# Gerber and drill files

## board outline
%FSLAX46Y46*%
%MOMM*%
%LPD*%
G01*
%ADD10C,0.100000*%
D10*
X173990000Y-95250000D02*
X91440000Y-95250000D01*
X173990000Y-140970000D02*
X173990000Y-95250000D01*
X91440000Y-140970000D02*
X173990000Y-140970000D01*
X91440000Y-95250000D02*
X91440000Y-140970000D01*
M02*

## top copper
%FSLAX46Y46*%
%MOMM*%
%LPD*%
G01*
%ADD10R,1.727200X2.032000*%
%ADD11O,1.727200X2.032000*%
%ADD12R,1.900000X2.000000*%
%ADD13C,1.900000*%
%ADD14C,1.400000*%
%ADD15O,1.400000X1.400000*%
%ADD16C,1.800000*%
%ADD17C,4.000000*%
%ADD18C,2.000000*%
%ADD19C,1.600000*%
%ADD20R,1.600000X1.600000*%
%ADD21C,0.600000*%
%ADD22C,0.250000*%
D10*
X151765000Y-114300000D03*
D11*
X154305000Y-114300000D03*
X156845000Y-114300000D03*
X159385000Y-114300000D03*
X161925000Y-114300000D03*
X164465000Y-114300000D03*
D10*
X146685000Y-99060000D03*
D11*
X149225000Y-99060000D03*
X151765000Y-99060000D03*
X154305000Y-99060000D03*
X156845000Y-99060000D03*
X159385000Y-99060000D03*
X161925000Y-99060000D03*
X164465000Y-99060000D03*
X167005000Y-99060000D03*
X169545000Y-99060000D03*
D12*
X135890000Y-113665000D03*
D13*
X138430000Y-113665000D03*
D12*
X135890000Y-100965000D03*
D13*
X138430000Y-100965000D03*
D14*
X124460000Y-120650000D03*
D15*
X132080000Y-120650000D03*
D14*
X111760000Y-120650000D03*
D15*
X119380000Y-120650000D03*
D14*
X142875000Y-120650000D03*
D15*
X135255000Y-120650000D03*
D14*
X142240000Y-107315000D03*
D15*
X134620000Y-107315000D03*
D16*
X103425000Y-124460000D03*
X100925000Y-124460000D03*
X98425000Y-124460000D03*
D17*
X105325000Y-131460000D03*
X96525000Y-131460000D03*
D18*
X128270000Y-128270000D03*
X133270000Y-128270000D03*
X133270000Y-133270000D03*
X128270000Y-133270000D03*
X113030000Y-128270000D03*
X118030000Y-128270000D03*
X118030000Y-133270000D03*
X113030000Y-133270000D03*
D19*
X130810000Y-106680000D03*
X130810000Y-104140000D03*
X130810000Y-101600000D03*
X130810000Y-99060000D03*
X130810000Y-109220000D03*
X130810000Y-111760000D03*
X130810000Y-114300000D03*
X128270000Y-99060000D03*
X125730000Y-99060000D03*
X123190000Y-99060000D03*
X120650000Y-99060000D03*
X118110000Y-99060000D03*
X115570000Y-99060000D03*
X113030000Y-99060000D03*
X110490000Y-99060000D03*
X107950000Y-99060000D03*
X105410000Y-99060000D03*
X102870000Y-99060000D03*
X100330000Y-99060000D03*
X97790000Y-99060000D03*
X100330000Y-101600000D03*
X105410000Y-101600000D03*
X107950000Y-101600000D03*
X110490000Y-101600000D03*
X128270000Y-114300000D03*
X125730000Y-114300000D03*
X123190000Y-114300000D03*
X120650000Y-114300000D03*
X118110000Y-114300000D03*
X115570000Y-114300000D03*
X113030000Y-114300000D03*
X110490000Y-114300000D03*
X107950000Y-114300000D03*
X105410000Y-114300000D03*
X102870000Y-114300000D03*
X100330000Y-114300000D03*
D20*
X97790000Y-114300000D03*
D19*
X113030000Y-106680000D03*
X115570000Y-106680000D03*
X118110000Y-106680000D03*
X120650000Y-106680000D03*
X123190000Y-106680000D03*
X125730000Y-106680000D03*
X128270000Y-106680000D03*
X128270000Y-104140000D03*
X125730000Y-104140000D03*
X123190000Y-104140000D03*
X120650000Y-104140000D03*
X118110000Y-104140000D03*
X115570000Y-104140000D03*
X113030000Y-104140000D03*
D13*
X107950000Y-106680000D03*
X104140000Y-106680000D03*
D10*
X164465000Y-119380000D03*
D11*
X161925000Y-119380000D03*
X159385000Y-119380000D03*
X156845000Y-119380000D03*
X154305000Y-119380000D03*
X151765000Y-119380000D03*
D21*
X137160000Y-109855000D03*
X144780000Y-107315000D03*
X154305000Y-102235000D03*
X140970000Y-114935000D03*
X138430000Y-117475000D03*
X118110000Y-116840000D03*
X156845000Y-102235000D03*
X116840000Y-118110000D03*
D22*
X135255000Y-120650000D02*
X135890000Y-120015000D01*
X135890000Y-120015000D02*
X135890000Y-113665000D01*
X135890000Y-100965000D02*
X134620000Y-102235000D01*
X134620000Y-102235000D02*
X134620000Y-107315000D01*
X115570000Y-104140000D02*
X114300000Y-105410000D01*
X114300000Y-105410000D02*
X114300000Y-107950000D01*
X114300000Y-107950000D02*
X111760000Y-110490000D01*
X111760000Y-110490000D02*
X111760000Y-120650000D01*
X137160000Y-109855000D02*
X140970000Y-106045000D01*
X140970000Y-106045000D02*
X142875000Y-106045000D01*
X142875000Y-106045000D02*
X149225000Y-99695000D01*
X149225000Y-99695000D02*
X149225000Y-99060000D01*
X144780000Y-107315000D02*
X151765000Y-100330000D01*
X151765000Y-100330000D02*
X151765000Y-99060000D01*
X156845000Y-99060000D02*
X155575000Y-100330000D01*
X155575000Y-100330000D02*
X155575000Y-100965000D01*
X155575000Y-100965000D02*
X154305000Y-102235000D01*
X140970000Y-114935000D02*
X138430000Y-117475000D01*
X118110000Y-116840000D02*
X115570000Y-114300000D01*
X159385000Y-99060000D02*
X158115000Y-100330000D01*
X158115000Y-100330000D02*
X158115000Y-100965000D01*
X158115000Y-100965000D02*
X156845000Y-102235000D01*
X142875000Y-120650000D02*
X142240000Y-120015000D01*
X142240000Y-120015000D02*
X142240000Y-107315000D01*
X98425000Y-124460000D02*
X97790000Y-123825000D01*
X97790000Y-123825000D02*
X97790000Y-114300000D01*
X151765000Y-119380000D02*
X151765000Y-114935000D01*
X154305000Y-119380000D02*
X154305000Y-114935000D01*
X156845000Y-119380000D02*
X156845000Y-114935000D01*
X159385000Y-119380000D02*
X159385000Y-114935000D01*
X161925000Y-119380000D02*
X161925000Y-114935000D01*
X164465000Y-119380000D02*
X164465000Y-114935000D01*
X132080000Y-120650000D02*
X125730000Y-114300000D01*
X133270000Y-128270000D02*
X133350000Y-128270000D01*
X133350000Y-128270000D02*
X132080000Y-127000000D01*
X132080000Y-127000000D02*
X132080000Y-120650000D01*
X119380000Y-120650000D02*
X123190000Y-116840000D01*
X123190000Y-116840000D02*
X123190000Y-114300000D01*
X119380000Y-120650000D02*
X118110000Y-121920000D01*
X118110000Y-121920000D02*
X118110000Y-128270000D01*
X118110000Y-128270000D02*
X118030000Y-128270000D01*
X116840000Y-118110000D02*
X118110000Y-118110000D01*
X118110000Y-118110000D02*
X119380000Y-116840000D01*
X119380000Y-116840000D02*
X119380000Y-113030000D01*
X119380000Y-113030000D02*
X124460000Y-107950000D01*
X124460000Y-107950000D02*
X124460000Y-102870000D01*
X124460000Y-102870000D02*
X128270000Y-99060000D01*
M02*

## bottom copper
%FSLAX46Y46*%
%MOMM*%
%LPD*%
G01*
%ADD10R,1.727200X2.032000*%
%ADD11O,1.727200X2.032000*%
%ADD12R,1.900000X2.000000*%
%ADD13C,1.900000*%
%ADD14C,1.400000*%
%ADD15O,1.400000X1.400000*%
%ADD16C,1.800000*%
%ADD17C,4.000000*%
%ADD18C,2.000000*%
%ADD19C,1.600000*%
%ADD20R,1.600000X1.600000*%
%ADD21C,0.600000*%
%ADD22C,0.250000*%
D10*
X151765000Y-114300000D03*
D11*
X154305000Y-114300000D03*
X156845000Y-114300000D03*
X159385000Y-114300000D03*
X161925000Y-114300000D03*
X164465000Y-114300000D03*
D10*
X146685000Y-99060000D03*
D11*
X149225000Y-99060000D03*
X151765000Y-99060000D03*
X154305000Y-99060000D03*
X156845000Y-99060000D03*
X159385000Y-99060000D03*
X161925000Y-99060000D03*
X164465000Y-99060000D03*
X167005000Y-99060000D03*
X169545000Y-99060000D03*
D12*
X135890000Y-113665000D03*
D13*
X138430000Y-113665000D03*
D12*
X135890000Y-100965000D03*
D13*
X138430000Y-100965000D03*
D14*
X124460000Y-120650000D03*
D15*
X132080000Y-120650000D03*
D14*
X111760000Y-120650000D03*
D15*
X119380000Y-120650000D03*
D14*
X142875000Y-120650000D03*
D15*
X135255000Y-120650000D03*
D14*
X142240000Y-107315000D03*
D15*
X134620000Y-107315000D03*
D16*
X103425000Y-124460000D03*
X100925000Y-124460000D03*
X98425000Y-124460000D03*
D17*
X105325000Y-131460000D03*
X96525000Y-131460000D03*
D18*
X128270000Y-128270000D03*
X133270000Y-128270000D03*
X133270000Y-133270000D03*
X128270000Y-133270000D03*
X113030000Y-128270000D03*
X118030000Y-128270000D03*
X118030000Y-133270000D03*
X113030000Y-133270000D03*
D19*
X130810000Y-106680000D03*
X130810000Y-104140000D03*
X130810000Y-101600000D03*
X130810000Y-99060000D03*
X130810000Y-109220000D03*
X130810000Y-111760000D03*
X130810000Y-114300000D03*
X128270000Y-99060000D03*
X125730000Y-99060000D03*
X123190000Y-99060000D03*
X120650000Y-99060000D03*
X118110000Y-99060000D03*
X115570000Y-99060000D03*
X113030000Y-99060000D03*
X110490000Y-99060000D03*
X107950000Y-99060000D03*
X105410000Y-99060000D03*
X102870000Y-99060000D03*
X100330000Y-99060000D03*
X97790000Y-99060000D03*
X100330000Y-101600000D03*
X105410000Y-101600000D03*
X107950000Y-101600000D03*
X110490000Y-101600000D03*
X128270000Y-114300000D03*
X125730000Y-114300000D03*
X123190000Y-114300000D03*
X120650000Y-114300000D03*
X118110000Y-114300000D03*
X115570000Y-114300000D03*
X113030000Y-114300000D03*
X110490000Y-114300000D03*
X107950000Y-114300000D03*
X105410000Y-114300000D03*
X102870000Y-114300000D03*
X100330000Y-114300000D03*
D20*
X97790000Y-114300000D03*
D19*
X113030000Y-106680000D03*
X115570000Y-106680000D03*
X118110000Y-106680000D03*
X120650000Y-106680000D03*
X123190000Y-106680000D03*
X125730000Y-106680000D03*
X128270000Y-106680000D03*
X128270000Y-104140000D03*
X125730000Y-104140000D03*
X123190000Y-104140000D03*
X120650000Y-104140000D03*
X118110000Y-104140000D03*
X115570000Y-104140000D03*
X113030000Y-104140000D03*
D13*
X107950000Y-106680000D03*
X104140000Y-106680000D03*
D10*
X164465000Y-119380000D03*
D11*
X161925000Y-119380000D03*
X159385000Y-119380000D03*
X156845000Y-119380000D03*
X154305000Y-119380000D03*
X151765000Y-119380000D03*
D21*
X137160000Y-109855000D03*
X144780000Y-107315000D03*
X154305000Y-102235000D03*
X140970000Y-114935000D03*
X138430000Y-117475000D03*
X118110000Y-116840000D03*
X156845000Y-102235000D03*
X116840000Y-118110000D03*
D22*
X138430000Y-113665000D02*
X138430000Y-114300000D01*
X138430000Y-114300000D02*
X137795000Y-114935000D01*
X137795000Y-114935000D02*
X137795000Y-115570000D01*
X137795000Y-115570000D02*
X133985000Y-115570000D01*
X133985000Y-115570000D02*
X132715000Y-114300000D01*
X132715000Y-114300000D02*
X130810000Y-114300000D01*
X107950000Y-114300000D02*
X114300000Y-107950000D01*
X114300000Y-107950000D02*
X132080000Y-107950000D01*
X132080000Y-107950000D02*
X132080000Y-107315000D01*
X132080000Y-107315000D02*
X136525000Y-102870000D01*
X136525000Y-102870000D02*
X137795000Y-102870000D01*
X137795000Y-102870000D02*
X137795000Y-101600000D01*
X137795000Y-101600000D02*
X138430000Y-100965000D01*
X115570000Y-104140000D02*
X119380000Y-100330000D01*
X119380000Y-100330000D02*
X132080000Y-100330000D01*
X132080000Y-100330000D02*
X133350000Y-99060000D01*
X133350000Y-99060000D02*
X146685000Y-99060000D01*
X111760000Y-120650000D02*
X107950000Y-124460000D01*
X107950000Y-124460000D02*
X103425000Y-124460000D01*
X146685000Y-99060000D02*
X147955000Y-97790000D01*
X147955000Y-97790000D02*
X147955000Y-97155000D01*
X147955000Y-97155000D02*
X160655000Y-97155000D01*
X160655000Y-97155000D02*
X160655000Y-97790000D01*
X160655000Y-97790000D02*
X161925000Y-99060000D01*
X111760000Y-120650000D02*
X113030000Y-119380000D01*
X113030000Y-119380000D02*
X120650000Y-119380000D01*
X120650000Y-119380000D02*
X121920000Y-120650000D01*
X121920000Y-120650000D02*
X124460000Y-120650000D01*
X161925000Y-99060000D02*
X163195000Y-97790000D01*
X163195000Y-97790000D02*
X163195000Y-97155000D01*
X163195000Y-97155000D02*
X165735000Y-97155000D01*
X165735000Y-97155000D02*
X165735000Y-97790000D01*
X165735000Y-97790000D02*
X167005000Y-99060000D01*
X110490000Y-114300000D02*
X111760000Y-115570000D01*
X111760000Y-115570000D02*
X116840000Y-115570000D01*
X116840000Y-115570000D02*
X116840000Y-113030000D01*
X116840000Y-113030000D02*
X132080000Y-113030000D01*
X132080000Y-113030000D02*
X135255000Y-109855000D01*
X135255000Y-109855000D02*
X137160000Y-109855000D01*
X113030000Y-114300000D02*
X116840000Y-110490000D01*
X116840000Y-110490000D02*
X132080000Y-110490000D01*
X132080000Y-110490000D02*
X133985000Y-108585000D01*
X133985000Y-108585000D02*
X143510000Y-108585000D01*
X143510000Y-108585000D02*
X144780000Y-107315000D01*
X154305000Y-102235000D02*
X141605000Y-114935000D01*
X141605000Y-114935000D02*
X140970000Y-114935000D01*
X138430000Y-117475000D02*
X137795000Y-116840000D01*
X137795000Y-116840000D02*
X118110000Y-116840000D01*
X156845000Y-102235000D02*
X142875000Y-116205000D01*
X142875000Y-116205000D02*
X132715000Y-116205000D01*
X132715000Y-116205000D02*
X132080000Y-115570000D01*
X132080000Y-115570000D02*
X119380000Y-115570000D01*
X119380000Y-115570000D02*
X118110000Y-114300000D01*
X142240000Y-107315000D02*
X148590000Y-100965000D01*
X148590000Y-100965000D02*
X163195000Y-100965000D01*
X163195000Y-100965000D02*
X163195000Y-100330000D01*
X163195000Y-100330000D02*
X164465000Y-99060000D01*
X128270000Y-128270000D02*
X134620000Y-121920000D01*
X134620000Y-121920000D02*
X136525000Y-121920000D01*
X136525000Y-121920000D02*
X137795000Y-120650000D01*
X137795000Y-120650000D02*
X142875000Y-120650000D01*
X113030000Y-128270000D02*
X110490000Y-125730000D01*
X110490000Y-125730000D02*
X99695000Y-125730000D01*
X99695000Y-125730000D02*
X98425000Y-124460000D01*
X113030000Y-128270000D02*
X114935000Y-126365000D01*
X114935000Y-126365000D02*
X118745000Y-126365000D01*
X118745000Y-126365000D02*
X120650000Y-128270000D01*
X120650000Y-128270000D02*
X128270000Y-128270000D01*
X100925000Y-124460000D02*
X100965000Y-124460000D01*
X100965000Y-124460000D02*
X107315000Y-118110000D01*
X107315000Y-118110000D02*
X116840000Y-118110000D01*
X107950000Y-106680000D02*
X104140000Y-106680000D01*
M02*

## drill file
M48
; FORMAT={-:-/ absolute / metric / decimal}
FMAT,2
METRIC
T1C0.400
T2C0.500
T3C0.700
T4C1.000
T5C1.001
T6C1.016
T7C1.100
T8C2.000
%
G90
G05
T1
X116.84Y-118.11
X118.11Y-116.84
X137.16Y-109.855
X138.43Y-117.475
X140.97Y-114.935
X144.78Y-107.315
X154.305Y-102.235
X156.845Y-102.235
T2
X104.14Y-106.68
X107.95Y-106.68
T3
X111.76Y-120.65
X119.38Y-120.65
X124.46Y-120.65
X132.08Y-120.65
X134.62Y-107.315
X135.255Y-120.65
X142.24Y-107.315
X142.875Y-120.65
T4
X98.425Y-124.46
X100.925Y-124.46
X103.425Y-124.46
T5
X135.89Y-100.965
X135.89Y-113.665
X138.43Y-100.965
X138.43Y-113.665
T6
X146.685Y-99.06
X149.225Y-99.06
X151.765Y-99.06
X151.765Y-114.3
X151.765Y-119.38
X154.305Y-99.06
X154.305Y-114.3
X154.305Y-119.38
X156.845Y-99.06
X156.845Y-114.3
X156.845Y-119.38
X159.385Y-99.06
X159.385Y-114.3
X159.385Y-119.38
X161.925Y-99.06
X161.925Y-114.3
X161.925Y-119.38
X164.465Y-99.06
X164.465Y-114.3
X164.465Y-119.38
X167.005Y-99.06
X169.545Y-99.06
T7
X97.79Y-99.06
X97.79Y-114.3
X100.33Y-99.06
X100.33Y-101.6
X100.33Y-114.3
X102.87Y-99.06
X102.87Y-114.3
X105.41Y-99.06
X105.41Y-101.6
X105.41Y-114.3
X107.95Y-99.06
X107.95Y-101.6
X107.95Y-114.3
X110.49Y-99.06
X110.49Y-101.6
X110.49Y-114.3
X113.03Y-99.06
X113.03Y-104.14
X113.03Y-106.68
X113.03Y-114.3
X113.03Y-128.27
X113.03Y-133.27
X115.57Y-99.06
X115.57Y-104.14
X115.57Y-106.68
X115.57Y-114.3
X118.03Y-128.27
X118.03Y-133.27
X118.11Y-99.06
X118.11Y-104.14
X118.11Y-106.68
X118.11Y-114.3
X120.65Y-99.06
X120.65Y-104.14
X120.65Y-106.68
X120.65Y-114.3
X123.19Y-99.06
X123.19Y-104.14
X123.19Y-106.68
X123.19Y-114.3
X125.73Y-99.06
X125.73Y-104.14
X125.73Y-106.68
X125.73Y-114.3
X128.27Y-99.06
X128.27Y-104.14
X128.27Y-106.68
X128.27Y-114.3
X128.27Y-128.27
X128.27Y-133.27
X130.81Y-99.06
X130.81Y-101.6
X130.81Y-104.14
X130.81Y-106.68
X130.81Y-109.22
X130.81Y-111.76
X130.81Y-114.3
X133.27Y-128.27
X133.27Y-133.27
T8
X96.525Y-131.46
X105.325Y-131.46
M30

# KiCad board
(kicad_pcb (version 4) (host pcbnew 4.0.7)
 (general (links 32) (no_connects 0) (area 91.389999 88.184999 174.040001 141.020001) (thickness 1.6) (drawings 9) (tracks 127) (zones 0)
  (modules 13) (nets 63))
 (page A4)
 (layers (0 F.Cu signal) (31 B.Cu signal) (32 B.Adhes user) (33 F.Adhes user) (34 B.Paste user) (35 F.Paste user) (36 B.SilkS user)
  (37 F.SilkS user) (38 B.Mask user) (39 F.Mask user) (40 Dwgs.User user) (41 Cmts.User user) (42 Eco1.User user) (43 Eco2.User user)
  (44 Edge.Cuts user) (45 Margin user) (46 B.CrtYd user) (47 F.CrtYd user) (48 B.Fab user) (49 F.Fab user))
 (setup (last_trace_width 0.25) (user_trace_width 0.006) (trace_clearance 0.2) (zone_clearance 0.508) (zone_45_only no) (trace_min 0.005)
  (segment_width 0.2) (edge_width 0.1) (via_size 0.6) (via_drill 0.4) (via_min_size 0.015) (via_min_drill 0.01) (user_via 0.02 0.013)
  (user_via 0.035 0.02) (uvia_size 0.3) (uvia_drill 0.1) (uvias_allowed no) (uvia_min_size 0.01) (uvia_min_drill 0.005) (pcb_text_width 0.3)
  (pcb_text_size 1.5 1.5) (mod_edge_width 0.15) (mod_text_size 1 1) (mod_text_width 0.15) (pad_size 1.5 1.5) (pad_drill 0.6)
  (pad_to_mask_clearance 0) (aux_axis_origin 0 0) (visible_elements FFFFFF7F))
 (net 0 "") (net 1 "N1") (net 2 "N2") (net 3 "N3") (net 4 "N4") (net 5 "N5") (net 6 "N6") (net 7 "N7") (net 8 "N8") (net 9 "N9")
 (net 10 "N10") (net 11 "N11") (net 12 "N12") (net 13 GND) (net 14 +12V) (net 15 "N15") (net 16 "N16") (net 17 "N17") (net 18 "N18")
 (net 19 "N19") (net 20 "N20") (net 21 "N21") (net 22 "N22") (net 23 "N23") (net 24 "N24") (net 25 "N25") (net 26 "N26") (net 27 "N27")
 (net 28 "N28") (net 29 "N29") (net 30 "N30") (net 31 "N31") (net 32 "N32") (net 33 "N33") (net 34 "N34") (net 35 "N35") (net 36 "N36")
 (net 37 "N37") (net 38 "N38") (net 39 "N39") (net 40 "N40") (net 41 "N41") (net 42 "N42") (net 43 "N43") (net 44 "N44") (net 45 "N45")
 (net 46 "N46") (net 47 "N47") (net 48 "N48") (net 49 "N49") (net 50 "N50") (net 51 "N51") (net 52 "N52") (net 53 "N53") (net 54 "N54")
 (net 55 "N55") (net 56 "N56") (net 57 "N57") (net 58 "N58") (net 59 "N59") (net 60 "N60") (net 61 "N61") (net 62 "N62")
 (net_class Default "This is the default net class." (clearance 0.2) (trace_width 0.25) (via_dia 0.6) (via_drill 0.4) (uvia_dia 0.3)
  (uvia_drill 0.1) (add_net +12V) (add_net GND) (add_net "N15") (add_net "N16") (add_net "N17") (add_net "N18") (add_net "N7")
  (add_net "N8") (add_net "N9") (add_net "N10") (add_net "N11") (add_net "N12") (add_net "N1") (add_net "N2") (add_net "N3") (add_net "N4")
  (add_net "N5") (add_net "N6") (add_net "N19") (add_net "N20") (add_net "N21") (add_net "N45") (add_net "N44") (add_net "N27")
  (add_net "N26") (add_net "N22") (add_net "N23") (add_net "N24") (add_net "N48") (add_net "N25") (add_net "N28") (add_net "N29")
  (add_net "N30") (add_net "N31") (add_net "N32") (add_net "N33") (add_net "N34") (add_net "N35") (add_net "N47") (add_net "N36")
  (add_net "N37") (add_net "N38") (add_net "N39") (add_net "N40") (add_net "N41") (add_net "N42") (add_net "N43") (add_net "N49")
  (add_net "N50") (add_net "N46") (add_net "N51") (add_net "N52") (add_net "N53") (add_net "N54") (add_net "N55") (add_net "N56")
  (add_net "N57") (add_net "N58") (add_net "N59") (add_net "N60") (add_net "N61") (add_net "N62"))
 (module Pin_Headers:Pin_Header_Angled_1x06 (layer F.Cu) (at 151.765 114.3 90)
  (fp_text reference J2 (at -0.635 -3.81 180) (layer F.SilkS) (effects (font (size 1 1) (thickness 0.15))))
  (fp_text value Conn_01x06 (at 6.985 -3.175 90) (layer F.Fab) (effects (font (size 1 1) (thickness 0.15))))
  (pad 1 thru_hole rect (at 0 0 90) (size 2.032 1.7272) (drill 1.016) (layers *.Cu *.Mask) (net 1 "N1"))
  (pad 2 thru_hole oval (at 0 2.54 90) (size 2.032 1.7272) (drill 1.016) (layers *.Cu *.Mask) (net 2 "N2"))
  (pad 3 thru_hole oval (at 0 5.08 90) (size 2.032 1.7272) (drill 1.016) (layers *.Cu *.Mask) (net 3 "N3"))
  (pad 4 thru_hole oval (at 0 7.62 90) (size 2.032 1.7272) (drill 1.016) (layers *.Cu *.Mask) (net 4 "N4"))
  (pad 5 thru_hole oval (at 0 10.16 90) (size 2.032 1.7272) (drill 1.016) (layers *.Cu *.Mask) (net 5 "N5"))
  (pad 6 thru_hole oval (at 0 12.7 90) (size 2.032 1.7272) (drill 1.016) (layers *.Cu *.Mask) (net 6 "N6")))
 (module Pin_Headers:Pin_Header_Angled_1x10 (layer F.Cu) (at 146.685 99.06 90)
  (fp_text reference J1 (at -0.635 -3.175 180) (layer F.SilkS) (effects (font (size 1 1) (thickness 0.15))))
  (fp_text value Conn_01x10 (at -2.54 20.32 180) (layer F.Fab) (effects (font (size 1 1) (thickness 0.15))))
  (pad 1 thru_hole rect (at 0 0 90) (size 2.032 1.7272) (drill 1.016) (layers *.Cu *.Mask) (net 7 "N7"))
  (pad 2 thru_hole oval (at 0 2.54 90) (size 2.032 1.7272) (drill 1.016) (layers *.Cu *.Mask) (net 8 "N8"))
  (pad 3 thru_hole oval (at 0 5.08 90) (size 2.032 1.7272) (drill 1.016) (layers *.Cu *.Mask) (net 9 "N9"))
  (pad 4 thru_hole oval (at 0 7.62 90) (size 2.032 1.7272) (drill 1.016) (layers *.Cu *.Mask) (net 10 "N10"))
  (pad 5 thru_hole oval (at 0 10.16 90) (size 2.032 1.7272) (drill 1.016) (layers *.Cu *.Mask) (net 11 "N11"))
  (pad 6 thru_hole oval (at 0 12.7 90) (size 2.032 1.7272) (drill 1.016) (layers *.Cu *.Mask) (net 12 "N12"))
  (pad 7 thru_hole oval (at 0 15.24 90) (size 2.032 1.7272) (drill 1.016) (layers *.Cu *.Mask) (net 7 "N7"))
  (pad 8 thru_hole oval (at 0 17.78 90) (size 2.032 1.7272) (drill 1.016) (layers *.Cu *.Mask) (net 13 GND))
  (pad 9 thru_hole oval (at 0 20.32 90) (size 2.032 1.7272) (drill 1.016) (layers *.Cu *.Mask) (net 7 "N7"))
  (pad 10 thru_hole oval (at 0 22.86 90) (size 2.032 1.7272) (drill 1.016) (layers *.Cu *.Mask) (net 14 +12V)))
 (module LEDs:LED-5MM (layer F.Cu) (at 135.89 113.665)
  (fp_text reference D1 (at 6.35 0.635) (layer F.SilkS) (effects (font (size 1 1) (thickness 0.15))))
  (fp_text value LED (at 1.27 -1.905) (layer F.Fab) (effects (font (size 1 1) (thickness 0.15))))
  (pad 1 thru_hole rect (at 0 0 90) (size 2 1.9) (drill 1.00076) (layers *.Cu *.Mask) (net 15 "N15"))
  (pad 2 thru_hole circle (at 2.54 0) (size 1.9 1.9) (drill 1.00076) (layers *.Cu *.Mask) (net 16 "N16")))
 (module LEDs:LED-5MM (layer F.Cu) (at 135.89 100.965)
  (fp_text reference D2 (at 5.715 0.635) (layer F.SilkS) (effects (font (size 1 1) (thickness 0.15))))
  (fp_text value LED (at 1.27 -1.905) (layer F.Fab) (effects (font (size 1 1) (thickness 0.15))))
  (pad 1 thru_hole rect (at 0 0 90) (size 2 1.9) (drill 1.00076) (layers *.Cu *.Mask) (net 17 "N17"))
  (pad 2 thru_hole circle (at 2.54 0) (size 1.9 1.9) (drill 1.00076) (layers *.Cu *.Mask) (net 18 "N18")))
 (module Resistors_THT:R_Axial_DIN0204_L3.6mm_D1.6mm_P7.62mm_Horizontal (layer F.Cu) (at 124.46 120.65)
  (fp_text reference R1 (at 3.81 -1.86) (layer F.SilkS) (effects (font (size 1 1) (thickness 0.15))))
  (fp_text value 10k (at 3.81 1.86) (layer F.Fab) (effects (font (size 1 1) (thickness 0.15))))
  (pad 1 thru_hole circle (at 0 0) (size 1.4 1.4) (drill 0.7) (layers *.Cu *.Mask) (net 7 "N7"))
  (pad 2 thru_hole oval (at 7.62 0) (size 1.4 1.4) (drill 0.7) (layers *.Cu *.Mask) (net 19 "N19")))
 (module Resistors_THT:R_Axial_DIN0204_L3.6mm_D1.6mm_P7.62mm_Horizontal (layer F.Cu) (at 111.76 120.65)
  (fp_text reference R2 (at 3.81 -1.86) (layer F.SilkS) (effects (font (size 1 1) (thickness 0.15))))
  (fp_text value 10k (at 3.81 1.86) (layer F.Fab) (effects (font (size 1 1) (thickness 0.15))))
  (pad 1 thru_hole circle (at 0 0) (size 1.4 1.4) (drill 0.7) (layers *.Cu *.Mask) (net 7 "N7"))
  (pad 2 thru_hole oval (at 7.62 0) (size 1.4 1.4) (drill 0.7) (layers *.Cu *.Mask) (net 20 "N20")))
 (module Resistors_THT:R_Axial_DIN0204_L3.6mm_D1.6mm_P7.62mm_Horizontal (layer F.Cu) (at 142.875 120.65 180)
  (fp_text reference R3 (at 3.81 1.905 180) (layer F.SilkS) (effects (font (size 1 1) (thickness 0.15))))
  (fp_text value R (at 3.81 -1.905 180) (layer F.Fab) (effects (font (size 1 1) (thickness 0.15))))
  (pad 1 thru_hole circle (at 0 0 180) (size 1.4 1.4) (drill 0.7) (layers *.Cu *.Mask) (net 13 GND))
  (pad 2 thru_hole oval (at 7.62 0 180) (size 1.4 1.4) (drill 0.7) (layers *.Cu *.Mask) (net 15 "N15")))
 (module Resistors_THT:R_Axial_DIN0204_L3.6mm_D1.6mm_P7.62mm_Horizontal (layer F.Cu) (at 142.24 107.315 180)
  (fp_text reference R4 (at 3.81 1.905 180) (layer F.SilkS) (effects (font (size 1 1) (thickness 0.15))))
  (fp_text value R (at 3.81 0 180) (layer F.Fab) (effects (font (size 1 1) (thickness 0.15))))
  (pad 1 thru_hole circle (at 0 0 180) (size 1.4 1.4) (drill 0.7) (layers *.Cu *.Mask) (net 13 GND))
  (pad 2 thru_hole oval (at 7.62 0 180) (size 1.4 1.4) (drill 0.7) (layers *.Cu *.Mask) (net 17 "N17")))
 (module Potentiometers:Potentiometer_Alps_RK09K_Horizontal (layer F.Cu) (at 98.425 124.46 270)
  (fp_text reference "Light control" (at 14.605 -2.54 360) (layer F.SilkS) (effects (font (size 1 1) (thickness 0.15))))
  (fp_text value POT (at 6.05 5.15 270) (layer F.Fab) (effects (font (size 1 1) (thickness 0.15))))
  (pad 3 thru_hole circle (at 0 -5 270) (size 1.8 1.8) (drill 1) (layers *.Cu *.Mask) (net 7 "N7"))
  (pad 2 thru_hole circle (at 0 -2.5 270) (size 1.8 1.8) (drill 1) (layers *.Cu *.Mask) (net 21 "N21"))
  (pad 1 thru_hole circle (at 0 0 270) (size 1.8 1.8) (drill 1) (layers *.Cu *.Mask) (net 13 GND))
  (pad 0 np_thru_hole circle (at 7 -6.9 270) (size 4 4) (drill 2) (layers *.Cu *.Mask))
  (pad 0 np_thru_hole circle (at 7 1.9 270) (size 4 4) (drill 2) (layers *.Cu *.Mask)))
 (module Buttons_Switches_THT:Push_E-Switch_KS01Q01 (layer F.Cu) (at 128.27 128.27)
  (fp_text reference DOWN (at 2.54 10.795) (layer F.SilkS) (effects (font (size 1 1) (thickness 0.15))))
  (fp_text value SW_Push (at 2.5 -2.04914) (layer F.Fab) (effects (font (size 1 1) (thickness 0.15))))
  (pad 1 thru_hole circle (at 0 0) (size 2 2) (drill 1.1) (layers *.Cu *.Mask) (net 13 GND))
  (pad 2 thru_hole circle (at 5 0) (size 2 2) (drill 1.1) (layers *.Cu *.Mask) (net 19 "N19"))
  (pad 4 thru_hole circle (at 5 5) (size 2 2) (drill 1.1) (layers *.Cu *.Mask))
  (pad 3 thru_hole circle (at 0 5) (size 2 2) (drill 1.1) (layers *.Cu *.Mask)))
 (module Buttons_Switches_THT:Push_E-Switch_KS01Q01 (layer F.Cu) (at 113.03 128.27)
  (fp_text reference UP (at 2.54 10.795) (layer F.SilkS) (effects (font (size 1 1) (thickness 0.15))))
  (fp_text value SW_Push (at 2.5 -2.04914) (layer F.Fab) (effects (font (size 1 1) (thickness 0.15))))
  (pad 1 thru_hole circle (at 0 0) (size 2 2) (drill 1.1) (layers *.Cu *.Mask) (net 13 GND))
  (pad 2 thru_hole circle (at 5 0) (size 2 2) (drill 1.1) (layers *.Cu *.Mask) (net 20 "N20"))
  (pad 4 thru_hole circle (at 5 5) (size 2 2) (drill 1.1) (layers *.Cu *.Mask))
  (pad 3 thru_hole circle (at 0 5) (size 2 2) (drill 1.1) (layers *.Cu *.Mask)))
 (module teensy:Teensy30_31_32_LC (layer F.Cu) (at 114.3 106.68)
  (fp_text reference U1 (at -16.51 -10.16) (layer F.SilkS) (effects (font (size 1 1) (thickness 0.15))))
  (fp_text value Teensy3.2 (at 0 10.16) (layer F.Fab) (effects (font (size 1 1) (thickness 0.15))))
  (pad 17 thru_hole circle (at 16.51 0) (size 1.6 1.6) (drill 1.1) (layers *.Cu *.Mask F.SilkS) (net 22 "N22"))
  (pad 18 thru_hole circle (at 16.51 -2.54) (size 1.6 1.6) (drill 1.1) (layers *.Cu *.Mask F.SilkS) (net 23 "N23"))
  (pad 19 thru_hole circle (at 16.51 -5.08) (size 1.6 1.6) (drill 1.1) (layers *.Cu *.Mask F.SilkS) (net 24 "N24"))
  (pad 20 thru_hole circle (at 16.51 -7.62) (size 1.6 1.6) (drill 1.1) (layers *.Cu *.Mask F.SilkS) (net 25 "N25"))
  (pad 16 thru_hole circle (at 16.51 2.54) (size 1.6 1.6) (drill 1.1) (layers *.Cu *.Mask F.SilkS) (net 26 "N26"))
  (pad 15 thru_hole circle (at 16.51 5.08) (size 1.6 1.6) (drill 1.1) (layers *.Cu *.Mask F.SilkS) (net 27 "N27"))
  (pad 14 thru_hole circle (at 16.51 7.62) (size 1.6 1.6) (drill 1.1) (layers *.Cu *.Mask F.SilkS) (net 16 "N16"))
  (pad 21 thru_hole circle (at 13.97 -7.62) (size 1.6 1.6) (drill 1.1) (layers *.Cu *.Mask F.SilkS) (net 21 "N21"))
  (pad 22 thru_hole circle (at 11.43 -7.62) (size 1.6 1.6) (drill 1.1) (layers *.Cu *.Mask F.SilkS) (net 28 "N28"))
  (pad 23 thru_hole circle (at 8.89 -7.62) (size 1.6 1.6) (drill 1.1) (layers *.Cu *.Mask F.SilkS) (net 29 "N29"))
  (pad 24 thru_hole circle (at 6.35 -7.62) (size 1.6 1.6) (drill 1.1) (layers *.Cu *.Mask F.SilkS) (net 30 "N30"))
  (pad 25 thru_hole circle (at 3.81 -7.62) (size 1.6 1.6) (drill 1.1) (layers *.Cu *.Mask F.SilkS) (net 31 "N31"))
  (pad 26 thru_hole circle (at 1.27 -7.62) (size 1.6 1.6) (drill 1.1) (layers *.Cu *.Mask F.SilkS) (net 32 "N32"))
  (pad 27 thru_hole circle (at -1.27 -7.62) (size 1.6 1.6) (drill 1.1) (layers *.Cu *.Mask F.SilkS) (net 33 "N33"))
  (pad 28 thru_hole circle (at -3.81 -7.62) (size 1.6 1.6) (drill 1.1) (layers *.Cu *.Mask F.SilkS) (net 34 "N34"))
  (pad 29 thru_hole circle (at -6.35 -7.62) (size 1.6 1.6) (drill 1.1) (layers *.Cu *.Mask F.SilkS) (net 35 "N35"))
  (pad 30 thru_hole circle (at -8.89 -7.62) (size 1.6 1.6) (drill 1.1) (layers *.Cu *.Mask F.SilkS) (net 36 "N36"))
  (pad 31 thru_hole circle (at -11.43 -7.62) (size 1.6 1.6) (drill 1.1) (layers *.Cu *.Mask F.SilkS) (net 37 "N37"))
  (pad 32 thru_hole circle (at -13.97 -7.62) (size 1.6 1.6) (drill 1.1) (layers *.Cu *.Mask F.SilkS) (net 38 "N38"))
  (pad 33 thru_hole circle (at -16.51 -7.62) (size 1.6 1.6) (drill 1.1) (layers *.Cu *.Mask F.SilkS) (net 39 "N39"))
  (pad 34 thru_hole circle (at -13.97 -5.08) (size 1.6 1.6) (drill 1.1) (layers *.Cu *.Mask F.SilkS) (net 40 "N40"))
  (pad 35 thru_hole circle (at -8.89 -5.08) (size 1.6 1.6) (drill 1.1) (layers *.Cu *.Mask F.SilkS) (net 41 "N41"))
  (pad 36 thru_hole circle (at -6.35 -5.08) (size 1.6 1.6) (drill 1.1) (layers *.Cu *.Mask F.SilkS) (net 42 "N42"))
  (pad 37 thru_hole circle (at -3.81 -5.08) (size 1.6 1.6) (drill 1.1) (layers *.Cu *.Mask F.SilkS) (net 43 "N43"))
  (pad 13 thru_hole circle (at 13.97 7.62) (size 1.6 1.6) (drill 1.1) (layers *.Cu *.Mask F.SilkS) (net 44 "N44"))
  (pad 12 thru_hole circle (at 11.43 7.62) (size 1.6 1.6) (drill 1.1) (layers *.Cu *.Mask F.SilkS) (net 19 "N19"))
  (pad 11 thru_hole circle (at 8.89 7.62) (size 1.6 1.6) (drill 1.1) (layers *.Cu *.Mask F.SilkS) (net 20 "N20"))
  (pad 10 thru_hole circle (at 6.35 7.62) (size 1.6 1.6) (drill 1.1) (layers *.Cu *.Mask F.SilkS) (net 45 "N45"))
  (pad 9 thru_hole circle (at 3.81 7.62) (size 1.6 1.6) (drill 1.1) (layers *.Cu *.Mask F.SilkS) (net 12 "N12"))
  (pad 8 thru_hole circle (at 1.27 7.62) (size 1.6 1.6) (drill 1.1) (layers *.Cu *.Mask F.SilkS) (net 11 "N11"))
  (pad 7 thru_hole circle (at -1.27 7.62) (size 1.6 1.6) (drill 1.1) (layers *.Cu *.Mask F.SilkS) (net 9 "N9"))
  (pad 6 thru_hole circle (at -3.81 7.62) (size 1.6 1.6) (drill 1.1) (layers *.Cu *.Mask F.SilkS) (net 8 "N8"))
  (pad 5 thru_hole circle (at -6.35 7.62) (size 1.6 1.6) (drill 1.1) (layers *.Cu *.Mask F.SilkS) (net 18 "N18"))
  (pad 4 thru_hole circle (at -8.89 7.62) (size 1.6 1.6) (drill 1.1) (layers *.Cu *.Mask F.SilkS) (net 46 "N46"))
  (pad 3 thru_hole circle (at -11.43 7.62) (size 1.6 1.6) (drill 1.1) (layers *.Cu *.Mask F.SilkS) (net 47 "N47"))
  (pad 2 thru_hole circle (at -13.97 7.62) (size 1.6 1.6) (drill 1.1) (layers *.Cu *.Mask F.SilkS) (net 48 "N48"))
  (pad 1 thru_hole rect (at -16.51 7.62) (size 1.6 1.6) (drill 1.1) (layers *.Cu *.Mask F.SilkS) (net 13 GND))
  (pad 38 thru_hole circle (at -1.27 0) (size 1.6 1.6) (drill 1.1) (layers *.Cu *.Mask) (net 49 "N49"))
  (pad 39 thru_hole circle (at 1.27 0) (size 1.6 1.6) (drill 1.1) (layers *.Cu *.Mask) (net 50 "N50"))
  (pad 40 thru_hole circle (at 3.81 0) (size 1.6 1.6) (drill 1.1) (layers *.Cu *.Mask) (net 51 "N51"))
  (pad 41 thru_hole circle (at 6.35 0) (size 1.6 1.6) (drill 1.1) (layers *.Cu *.Mask) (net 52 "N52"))
  (pad 42 thru_hole circle (at 8.89 0) (size 1.6 1.6) (drill 1.1) (layers *.Cu *.Mask) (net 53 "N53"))
  (pad 43 thru_hole circle (at 11.43 0) (size 1.6 1.6) (drill 1.1) (layers *.Cu *.Mask) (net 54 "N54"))
  (pad 44 thru_hole circle (at 13.97 0) (size 1.6 1.6) (drill 1.1) (layers *.Cu *.Mask) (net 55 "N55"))
  (pad 45 thru_hole circle (at 13.97 -2.54) (size 1.6 1.6) (drill 1.1) (layers *.Cu *.Mask) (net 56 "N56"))
  (pad 46 thru_hole circle (at 11.43 -2.54) (size 1.6 1.6) (drill 1.1) (layers *.Cu *.Mask) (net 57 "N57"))
  (pad 47 thru_hole circle (at 8.89 -2.54) (size 1.6 1.6) (drill 1.1) (layers *.Cu *.Mask) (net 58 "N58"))
  (pad 48 thru_hole circle (at 6.35 -2.54) (size 1.6 1.6) (drill 1.1) (layers *.Cu *.Mask) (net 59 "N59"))
  (pad 49 thru_hole circle (at 3.81 -2.54) (size 1.6 1.6) (drill 1.1) (layers *.Cu *.Mask) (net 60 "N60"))
  (pad 50 thru_hole circle (at 1.27 -2.54) (size 1.6 1.6) (drill 1.1) (layers *.Cu *.Mask) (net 7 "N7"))
  (pad 51 thru_hole circle (at -1.27 -2.54) (size 1.6 1.6) (drill 1.1) (layers *.Cu *.Mask) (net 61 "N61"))
  (pad 52 thru_hole circle (at -6.35 0) (size 1.9 1.9) (drill 0.5) (layers *.Cu *.Mask F.SilkS) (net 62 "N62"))
  (pad 52 thru_hole circle (at -10.16 0) (size 1.9 1.9) (drill 0.5) (layers *.Cu *.Mask F.SilkS) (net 62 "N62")))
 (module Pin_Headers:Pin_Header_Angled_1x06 (layer F.Cu) (at 164.465 119.38 270)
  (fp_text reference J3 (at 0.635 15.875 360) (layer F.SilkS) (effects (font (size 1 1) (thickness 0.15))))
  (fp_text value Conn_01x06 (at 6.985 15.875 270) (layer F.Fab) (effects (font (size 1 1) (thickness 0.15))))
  (pad 1 thru_hole rect (at 0 0 270) (size 2.032 1.7272) (drill 1.016) (layers *.Cu *.Mask) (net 6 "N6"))
  (pad 2 thru_hole oval (at 0 2.54 270) (size 2.032 1.7272) (drill 1.016) (layers *.Cu *.Mask) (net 5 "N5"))
  (pad 3 thru_hole oval (at 0 5.08 270) (size 2.032 1.7272) (drill 1.016) (layers *.Cu *.Mask) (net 4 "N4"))
  (pad 4 thru_hole oval (at 0 7.62 270) (size 2.032 1.7272) (drill 1.016) (layers *.Cu *.Mask) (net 3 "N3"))
  (pad 5 thru_hole oval (at 0 10.16 270) (size 2.032 1.7272) (drill 1.016) (layers *.Cu *.Mask) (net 2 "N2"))
  (pad 6 thru_hole oval (at 0 12.7 270) (size 2.032 1.7272) (drill 1.016) (layers *.Cu *.Mask) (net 1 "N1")))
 (gr_line (start 173.99 95.25) (end 91.44 95.25) (angle 90) (layer Edge.Cuts) (width 0.1))
 (gr_line (start 173.99 140.97) (end 173.99 95.25) (angle 90) (layer Edge.Cuts) (width 0.1))
 (gr_line (start 91.44 140.97) (end 173.99 140.97) (angle 90) (layer Edge.Cuts) (width 0.1))
 (gr_line (start 91.44 95.25) (end 91.44 140.97) (angle 90) (layer Edge.Cuts) (width 0.1))
 (segment (start 135.255 120.65) (end 135.89 120.015) (width 0.25) (layer F.Cu) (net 15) (status 80000))
 (segment (start 135.89 120.015) (end 135.89 113.665) (width 0.25) (layer F.Cu) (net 15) (status 80000))
 (segment (start 138.43 113.665) (end 138.43 114.3) (width 0.25) (layer B.Cu) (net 16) (status 80000))
 (segment (start 138.43 114.3) (end 137.795 114.935) (width 0.25) (layer B.Cu) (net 16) (status 80000))
 (segment (start 137.795 114.935) (end 137.795 115.57) (width 0.25) (layer B.Cu) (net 16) (status 80000))
 (segment (start 137.795 115.57) (end 133.985 115.57) (width 0.25) (layer B.Cu) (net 16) (status 80000))
 (segment (start 133.985 115.57) (end 132.715 114.3) (width 0.25) (layer B.Cu) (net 16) (status 80000))
 (segment (start 132.715 114.3) (end 130.81 114.3) (width 0.25) (layer B.Cu) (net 16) (status 80000))
 (segment (start 135.89 100.965) (end 134.62 102.235) (width 0.25) (layer F.Cu) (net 17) (status 80000))
 (segment (start 134.62 102.235) (end 134.62 107.315) (width 0.25) (layer F.Cu) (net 17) (status 80000))
 (segment (start 107.95 114.3) (end 114.3 107.95) (width 0.25) (layer B.Cu) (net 18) (status 80000))
 (segment (start 114.3 107.95) (end 132.08 107.95) (width 0.25) (layer B.Cu) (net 18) (status 80000))
 (segment (start 132.08 107.95) (end 132.08 107.315) (width 0.25) (layer B.Cu) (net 18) (status 80000))
 (segment (start 132.08 107.315) (end 136.525 102.87) (width 0.25) (layer B.Cu) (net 18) (status 80000))
 (segment (start 136.525 102.87) (end 137.795 102.87) (width 0.25) (layer B.Cu) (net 18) (status 80000))
 (segment (start 137.795 102.87) (end 137.795 101.6) (width 0.25) (layer B.Cu) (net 18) (status 80000))
 (segment (start 137.795 101.6) (end 138.43 100.965) (width 0.25) (layer B.Cu) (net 18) (status 80000))
 (segment (start 115.57 104.14) (end 119.38 100.33) (width 0.25) (layer B.Cu) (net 7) (status 80000))
 (segment (start 119.38 100.33) (end 132.08 100.33) (width 0.25) (layer B.Cu) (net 7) (status 80000))
 (segment (start 132.08 100.33) (end 133.35 99.06) (width 0.25) (layer B.Cu) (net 7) (status 80000))
 (segment (start 133.35 99.06) (end 146.685 99.06) (width 0.25) (layer B.Cu) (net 7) (status 80000))
 (segment (start 115.57 104.14) (end 114.3 105.41) (width 0.25) (layer F.Cu) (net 7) (status 80000))
 (segment (start 114.3 105.41) (end 114.3 107.95) (width 0.25) (layer F.Cu) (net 7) (status 80000))
 (segment (start 114.3 107.95) (end 111.76 110.49) (width 0.25) (layer F.Cu) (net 7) (status 80000))
 (segment (start 111.76 110.49) (end 111.76 120.65) (width 0.25) (layer F.Cu) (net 7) (status 80000))
 (segment (start 111.76 120.65) (end 107.95 124.46) (width 0.25) (layer B.Cu) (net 7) (status 80000))
 (segment (start 107.95 124.46) (end 103.425 124.46) (width 0.25) (layer B.Cu) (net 7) (status 80000))
 (segment (start 146.685 99.06) (end 147.955 97.79) (width 0.25) (layer B.Cu) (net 7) (status 80000))
 (segment (start 147.955 97.79) (end 147.955 97.155) (width 0.25) (layer B.Cu) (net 7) (status 80000))
 (segment (start 147.955 97.155) (end 160.655 97.155) (width 0.25) (layer B.Cu) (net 7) (status 80000))
 (segment (start 160.655 97.155) (end 160.655 97.79) (width 0.25) (layer B.Cu) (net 7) (status 80000))
 (segment (start 160.655 97.79) (end 161.925 99.06) (width 0.25) (layer B.Cu) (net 7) (status 80000))
 (segment (start 111.76 120.65) (end 113.03 119.38) (width 0.25) (layer B.Cu) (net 7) (status 80000))
 (segment (start 113.03 119.38) (end 120.65 119.38) (width 0.25) (layer B.Cu) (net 7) (status 80000))
 (segment (start 120.65 119.38) (end 121.92 120.65) (width 0.25) (layer B.Cu) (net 7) (status 80000))
 (segment (start 121.92 120.65) (end 124.46 120.65) (width 0.25) (layer B.Cu) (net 7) (status 80000))
 (segment (start 161.925 99.06) (end 163.195 97.79) (width 0.25) (layer B.Cu) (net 7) (status 80000))
 (segment (start 163.195 97.79) (end 163.195 97.155) (width 0.25) (layer B.Cu) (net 7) (status 80000))
 (segment (start 163.195 97.155) (end 165.735 97.155) (width 0.25) (layer B.Cu) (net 7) (status 80000))
 (segment (start 165.735 97.155) (end 165.735 97.79) (width 0.25) (layer B.Cu) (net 7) (status 80000))
 (segment (start 165.735 97.79) (end 167.005 99.06) (width 0.25) (layer B.Cu) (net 7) (status 80000))
 (segment (start 110.49 114.3) (end 111.76 115.57) (width 0.25) (layer B.Cu) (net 8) (status 80000))
 (segment (start 111.76 115.57) (end 116.84 115.57) (width 0.25) (layer B.Cu) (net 8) (status 80000))
 (segment (start 116.84 115.57) (end 116.84 113.03) (width 0.25) (layer B.Cu) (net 8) (status 80000))
 (segment (start 116.84 113.03) (end 132.08 113.03) (width 0.25) (layer B.Cu) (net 8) (status 80000))
 (segment (start 132.08 113.03) (end 135.255 109.855) (width 0.25) (layer B.Cu) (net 8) (status 80000))
 (segment (start 135.255 109.855) (end 137.16 109.855) (width 0.25) (layer B.Cu) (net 8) (status 80000))
 (via (at 137.16 109.855) (size 0.6) (layers F.Cu B.Cu) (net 8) (status 80000))
 (segment (start 137.16 109.855) (end 140.97 106.045) (width 0.25) (layer F.Cu) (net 8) (status 80000))
 (segment (start 140.97 106.045) (end 142.875 106.045) (width 0.25) (layer F.Cu) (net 8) (status 80000))
 (segment (start 142.875 106.045) (end 149.225 99.695) (width 0.25) (layer F.Cu) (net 8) (status 80000))
 (segment (start 149.225 99.695) (end 149.225 99.06) (width 0.25) (layer F.Cu) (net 8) (status 80000))
 (segment (start 113.03 114.3) (end 116.84 110.49) (width 0.25) (layer B.Cu) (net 9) (status 80000))
 (segment (start 116.84 110.49) (end 132.08 110.49) (width 0.25) (layer B.Cu) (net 9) (status 80000))
 (segment (start 132.08 110.49) (end 133.985 108.585) (width 0.25) (layer B.Cu) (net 9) (status 80000))
 (segment (start 133.985 108.585) (end 143.51 108.585) (width 0.25) (layer B.Cu) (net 9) (status 80000))
 (segment (start 143.51 108.585) (end 144.78 107.315) (width 0.25) (layer B.Cu) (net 9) (status 80000))
 (via (at 144.78 107.315) (size 0.6) (layers F.Cu B.Cu) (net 9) (status 80000))
 (segment (start 144.78 107.315) (end 151.765 100.33) (width 0.25) (layer F.Cu) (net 9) (status 80000))
 (segment (start 151.765 100.33) (end 151.765 99.06) (width 0.25) (layer F.Cu) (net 9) (status 80000))
 (segment (start 156.845 99.06) (end 155.575 100.33) (width 0.25) (layer F.Cu) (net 11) (status 80000))
 (segment (start 155.575 100.33) (end 155.575 100.965) (width 0.25) (layer F.Cu) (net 11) (status 80000))
 (segment (start 155.575 100.965) (end 154.305 102.235) (width 0.25) (layer F.Cu) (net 11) (status 80000))
 (via (at 154.305 102.235) (size 0.6) (layers F.Cu B.Cu) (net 11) (status 80000))
 (segment (start 154.305 102.235) (end 141.605 114.935) (width 0.25) (layer B.Cu) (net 11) (status 80000))
 (segment (start 141.605 114.935) (end 140.97 114.935) (width 0.25) (layer B.Cu) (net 11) (status 80000))
 (via (at 140.97 114.935) (size 0.6) (layers F.Cu B.Cu) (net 11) (status 80000))
 (segment (start 140.97 114.935) (end 138.43 117.475) (width 0.25) (layer F.Cu) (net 11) (status 80000))
 (via (at 138.43 117.475) (size 0.6) (layers F.Cu B.Cu) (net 11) (status 80000))
 (segment (start 138.43 117.475) (end 137.795 116.84) (width 0.25) (layer B.Cu) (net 11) (status 80000))
 (segment (start 137.795 116.84) (end 118.11 116.84) (width 0.25) (layer B.Cu) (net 11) (status 80000))
 (via (at 118.11 116.84) (size 0.6) (layers F.Cu B.Cu) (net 11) (status 80000))
 (segment (start 118.11 116.84) (end 115.57 114.3) (width 0.25) (layer F.Cu) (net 11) (status 80000))
 (segment (start 159.385 99.06) (end 158.115 100.33) (width 0.25) (layer F.Cu) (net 12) (status 80000))
 (segment (start 158.115 100.33) (end 158.115 100.965) (width 0.25) (layer F.Cu) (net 12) (status 80000))
 (segment (start 158.115 100.965) (end 156.845 102.235) (width 0.25) (layer F.Cu) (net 12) (status 80000))
 (via (at 156.845 102.235) (size 0.6) (layers F.Cu B.Cu) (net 12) (status 80000))
 (segment (start 156.845 102.235) (end 142.875 116.205) (width 0.25) (layer B.Cu) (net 12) (status 80000))
 (segment (start 142.875 116.205) (end 132.715 116.205) (width 0.25) (layer B.Cu) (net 12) (status 80000))
 (segment (start 132.715 116.205) (end 132.08 115.57) (width 0.25) (layer B.Cu) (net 12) (status 80000))
 (segment (start 132.08 115.57) (end 119.38 115.57) (width 0.25) (layer B.Cu) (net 12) (status 80000))
 (segment (start 119.38 115.57) (end 118.11 114.3) (width 0.25) (layer B.Cu) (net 12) (status 80000))
 (segment (start 142.24 107.315) (end 148.59 100.965) (width 0.25) (layer B.Cu) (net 13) (status 80000))
 (segment (start 148.59 100.965) (end 163.195 100.965) (width 0.25) (layer B.Cu) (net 13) (status 80000))
 (segment (start 163.195 100.965) (end 163.195 100.33) (width 0.25) (layer B.Cu) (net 13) (status 80000))
 (segment (start 163.195 100.33) (end 164.465 99.06) (width 0.25) (layer B.Cu) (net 13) (status 80000))
 (segment (start 128.27 128.27) (end 134.62 121.92) (width 0.25) (layer B.Cu) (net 13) (status 80000))
 (segment (start 134.62 121.92) (end 136.525 121.92) (width 0.25) (layer B.Cu) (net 13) (status 80000))
 (segment (start 136.525 121.92) (end 137.795 120.65) (width 0.25) (layer B.Cu) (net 13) (status 80000))
 (segment (start 137.795 120.65) (end 142.875 120.65) (width 0.25) (layer B.Cu) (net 13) (status 80000))
 (segment (start 113.03 128.27) (end 110.49 125.73) (width 0.25) (layer B.Cu) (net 13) (status 80000))
 (segment (start 110.49 125.73) (end 99.695 125.73) (width 0.25) (layer B.Cu) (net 13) (status 80000))
 (segment (start 99.695 125.73) (end 98.425 124.46) (width 0.25) (layer B.Cu) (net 13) (status 80000))
 (segment (start 113.03 128.27) (end 114.935 126.365) (width 0.25) (layer B.Cu) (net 13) (status 80000))
 (segment (start 114.935 126.365) (end 118.745 126.365) (width 0.25) (layer B.Cu) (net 13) (status 80000))
 (segment (start 118.745 126.365) (end 120.65 128.27) (width 0.25) (layer B.Cu) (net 13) (status 80000))
 (segment (start 120.65 128.27) (end 128.27 128.27) (width 0.25) (layer B.Cu) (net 13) (status 80000))
 (segment (start 142.875 120.65) (end 142.24 120.015) (width 0.25) (layer F.Cu) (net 13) (status 80000))
 (segment (start 142.24 120.015) (end 142.24 107.315) (width 0.25) (layer F.Cu) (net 13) (status 80000))
 (segment (start 98.425 124.46) (end 97.79 123.825) (width 0.25) (layer F.Cu) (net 13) (status 80000))
 (segment (start 97.79 123.825) (end 97.79 114.3) (width 0.25) (layer F.Cu) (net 13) (status 80000))
 (segment (start 151.765 119.38) (end 151.765 114.935) (width 0.25) (layer F.Cu) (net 1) (status 80000))
 (segment (start 154.305 119.38) (end 154.305 114.935) (width 0.25) (layer F.Cu) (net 2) (status 80000))
 (segment (start 156.845 119.38) (end 156.845 114.935) (width 0.25) (layer F.Cu) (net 3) (status 80000))
 (segment (start 159.385 119.38) (end 159.385 114.935) (width 0.25) (layer F.Cu) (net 4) (status 80000))
 (segment (start 161.925 119.38) (end 161.925 114.935) (width 0.25) (layer F.Cu) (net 5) (status 80000))
 (segment (start 164.465 119.38) (end 164.465 114.935) (width 0.25) (layer F.Cu) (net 6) (status 80000))
 (segment (start 132.08 120.65) (end 125.73 114.3) (width 0.25) (layer F.Cu) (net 19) (status 80000))
 (segment (start 133.27 128.27) (end 133.35 128.27) (width 0.25) (layer F.Cu) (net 19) (status 80000))
 (segment (start 133.35 128.27) (end 132.08 127) (width 0.25) (layer F.Cu) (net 19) (status 80000))
 (segment (start 132.08 127) (end 132.08 120.65) (width 0.25) (layer F.Cu) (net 19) (status 80000))
 (segment (start 119.38 120.65) (end 123.19 116.84) (width 0.25) (layer F.Cu) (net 20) (status 80000))
 (segment (start 123.19 116.84) (end 123.19 114.3) (width 0.25) (layer F.Cu) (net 20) (status 80000))
 (segment (start 119.38 120.65) (end 118.11 121.92) (width 0.25) (layer F.Cu) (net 20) (status 80000))
 (segment (start 118.11 121.92) (end 118.11 128.27) (width 0.25) (layer F.Cu) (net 20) (status 80000))
 (segment (start 118.11 128.27) (end 118.03 128.27) (width 0.25) (layer F.Cu) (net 20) (status 80000))
 (segment (start 100.925 124.46) (end 100.965 124.46) (width 0.25) (layer B.Cu) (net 21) (status 80000))
 (segment (start 100.965 124.46) (end 107.315 118.11) (width 0.25) (layer B.Cu) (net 21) (status 80000))
 (segment (start 107.315 118.11) (end 116.84 118.11) (width 0.25) (layer B.Cu) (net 21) (status 80000))
 (via (at 116.84 118.11) (size 0.6) (layers F.Cu B.Cu) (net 21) (status 80000))
 (segment (start 116.84 118.11) (end 118.11 118.11) (width 0.25) (layer F.Cu) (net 21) (status 80000))
 (segment (start 118.11 118.11) (end 119.38 116.84) (width 0.25) (layer F.Cu) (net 21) (status 80000))
 (segment (start 119.38 116.84) (end 119.38 113.03) (width 0.25) (layer F.Cu) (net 21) (status 80000))
 (segment (start 119.38 113.03) (end 124.46 107.95) (width 0.25) (layer F.Cu) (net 21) (status 80000))
 (segment (start 124.46 107.95) (end 124.46 102.87) (width 0.25) (layer F.Cu) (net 21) (status 80000))
 (segment (start 124.46 102.87) (end 128.27 99.06) (width 0.25) (layer F.Cu) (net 21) (status 80000))
 (segment (start 107.95 106.68) (end 104.14 106.68) (width 0.25) (layer B.Cu) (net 62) (status 80000)))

